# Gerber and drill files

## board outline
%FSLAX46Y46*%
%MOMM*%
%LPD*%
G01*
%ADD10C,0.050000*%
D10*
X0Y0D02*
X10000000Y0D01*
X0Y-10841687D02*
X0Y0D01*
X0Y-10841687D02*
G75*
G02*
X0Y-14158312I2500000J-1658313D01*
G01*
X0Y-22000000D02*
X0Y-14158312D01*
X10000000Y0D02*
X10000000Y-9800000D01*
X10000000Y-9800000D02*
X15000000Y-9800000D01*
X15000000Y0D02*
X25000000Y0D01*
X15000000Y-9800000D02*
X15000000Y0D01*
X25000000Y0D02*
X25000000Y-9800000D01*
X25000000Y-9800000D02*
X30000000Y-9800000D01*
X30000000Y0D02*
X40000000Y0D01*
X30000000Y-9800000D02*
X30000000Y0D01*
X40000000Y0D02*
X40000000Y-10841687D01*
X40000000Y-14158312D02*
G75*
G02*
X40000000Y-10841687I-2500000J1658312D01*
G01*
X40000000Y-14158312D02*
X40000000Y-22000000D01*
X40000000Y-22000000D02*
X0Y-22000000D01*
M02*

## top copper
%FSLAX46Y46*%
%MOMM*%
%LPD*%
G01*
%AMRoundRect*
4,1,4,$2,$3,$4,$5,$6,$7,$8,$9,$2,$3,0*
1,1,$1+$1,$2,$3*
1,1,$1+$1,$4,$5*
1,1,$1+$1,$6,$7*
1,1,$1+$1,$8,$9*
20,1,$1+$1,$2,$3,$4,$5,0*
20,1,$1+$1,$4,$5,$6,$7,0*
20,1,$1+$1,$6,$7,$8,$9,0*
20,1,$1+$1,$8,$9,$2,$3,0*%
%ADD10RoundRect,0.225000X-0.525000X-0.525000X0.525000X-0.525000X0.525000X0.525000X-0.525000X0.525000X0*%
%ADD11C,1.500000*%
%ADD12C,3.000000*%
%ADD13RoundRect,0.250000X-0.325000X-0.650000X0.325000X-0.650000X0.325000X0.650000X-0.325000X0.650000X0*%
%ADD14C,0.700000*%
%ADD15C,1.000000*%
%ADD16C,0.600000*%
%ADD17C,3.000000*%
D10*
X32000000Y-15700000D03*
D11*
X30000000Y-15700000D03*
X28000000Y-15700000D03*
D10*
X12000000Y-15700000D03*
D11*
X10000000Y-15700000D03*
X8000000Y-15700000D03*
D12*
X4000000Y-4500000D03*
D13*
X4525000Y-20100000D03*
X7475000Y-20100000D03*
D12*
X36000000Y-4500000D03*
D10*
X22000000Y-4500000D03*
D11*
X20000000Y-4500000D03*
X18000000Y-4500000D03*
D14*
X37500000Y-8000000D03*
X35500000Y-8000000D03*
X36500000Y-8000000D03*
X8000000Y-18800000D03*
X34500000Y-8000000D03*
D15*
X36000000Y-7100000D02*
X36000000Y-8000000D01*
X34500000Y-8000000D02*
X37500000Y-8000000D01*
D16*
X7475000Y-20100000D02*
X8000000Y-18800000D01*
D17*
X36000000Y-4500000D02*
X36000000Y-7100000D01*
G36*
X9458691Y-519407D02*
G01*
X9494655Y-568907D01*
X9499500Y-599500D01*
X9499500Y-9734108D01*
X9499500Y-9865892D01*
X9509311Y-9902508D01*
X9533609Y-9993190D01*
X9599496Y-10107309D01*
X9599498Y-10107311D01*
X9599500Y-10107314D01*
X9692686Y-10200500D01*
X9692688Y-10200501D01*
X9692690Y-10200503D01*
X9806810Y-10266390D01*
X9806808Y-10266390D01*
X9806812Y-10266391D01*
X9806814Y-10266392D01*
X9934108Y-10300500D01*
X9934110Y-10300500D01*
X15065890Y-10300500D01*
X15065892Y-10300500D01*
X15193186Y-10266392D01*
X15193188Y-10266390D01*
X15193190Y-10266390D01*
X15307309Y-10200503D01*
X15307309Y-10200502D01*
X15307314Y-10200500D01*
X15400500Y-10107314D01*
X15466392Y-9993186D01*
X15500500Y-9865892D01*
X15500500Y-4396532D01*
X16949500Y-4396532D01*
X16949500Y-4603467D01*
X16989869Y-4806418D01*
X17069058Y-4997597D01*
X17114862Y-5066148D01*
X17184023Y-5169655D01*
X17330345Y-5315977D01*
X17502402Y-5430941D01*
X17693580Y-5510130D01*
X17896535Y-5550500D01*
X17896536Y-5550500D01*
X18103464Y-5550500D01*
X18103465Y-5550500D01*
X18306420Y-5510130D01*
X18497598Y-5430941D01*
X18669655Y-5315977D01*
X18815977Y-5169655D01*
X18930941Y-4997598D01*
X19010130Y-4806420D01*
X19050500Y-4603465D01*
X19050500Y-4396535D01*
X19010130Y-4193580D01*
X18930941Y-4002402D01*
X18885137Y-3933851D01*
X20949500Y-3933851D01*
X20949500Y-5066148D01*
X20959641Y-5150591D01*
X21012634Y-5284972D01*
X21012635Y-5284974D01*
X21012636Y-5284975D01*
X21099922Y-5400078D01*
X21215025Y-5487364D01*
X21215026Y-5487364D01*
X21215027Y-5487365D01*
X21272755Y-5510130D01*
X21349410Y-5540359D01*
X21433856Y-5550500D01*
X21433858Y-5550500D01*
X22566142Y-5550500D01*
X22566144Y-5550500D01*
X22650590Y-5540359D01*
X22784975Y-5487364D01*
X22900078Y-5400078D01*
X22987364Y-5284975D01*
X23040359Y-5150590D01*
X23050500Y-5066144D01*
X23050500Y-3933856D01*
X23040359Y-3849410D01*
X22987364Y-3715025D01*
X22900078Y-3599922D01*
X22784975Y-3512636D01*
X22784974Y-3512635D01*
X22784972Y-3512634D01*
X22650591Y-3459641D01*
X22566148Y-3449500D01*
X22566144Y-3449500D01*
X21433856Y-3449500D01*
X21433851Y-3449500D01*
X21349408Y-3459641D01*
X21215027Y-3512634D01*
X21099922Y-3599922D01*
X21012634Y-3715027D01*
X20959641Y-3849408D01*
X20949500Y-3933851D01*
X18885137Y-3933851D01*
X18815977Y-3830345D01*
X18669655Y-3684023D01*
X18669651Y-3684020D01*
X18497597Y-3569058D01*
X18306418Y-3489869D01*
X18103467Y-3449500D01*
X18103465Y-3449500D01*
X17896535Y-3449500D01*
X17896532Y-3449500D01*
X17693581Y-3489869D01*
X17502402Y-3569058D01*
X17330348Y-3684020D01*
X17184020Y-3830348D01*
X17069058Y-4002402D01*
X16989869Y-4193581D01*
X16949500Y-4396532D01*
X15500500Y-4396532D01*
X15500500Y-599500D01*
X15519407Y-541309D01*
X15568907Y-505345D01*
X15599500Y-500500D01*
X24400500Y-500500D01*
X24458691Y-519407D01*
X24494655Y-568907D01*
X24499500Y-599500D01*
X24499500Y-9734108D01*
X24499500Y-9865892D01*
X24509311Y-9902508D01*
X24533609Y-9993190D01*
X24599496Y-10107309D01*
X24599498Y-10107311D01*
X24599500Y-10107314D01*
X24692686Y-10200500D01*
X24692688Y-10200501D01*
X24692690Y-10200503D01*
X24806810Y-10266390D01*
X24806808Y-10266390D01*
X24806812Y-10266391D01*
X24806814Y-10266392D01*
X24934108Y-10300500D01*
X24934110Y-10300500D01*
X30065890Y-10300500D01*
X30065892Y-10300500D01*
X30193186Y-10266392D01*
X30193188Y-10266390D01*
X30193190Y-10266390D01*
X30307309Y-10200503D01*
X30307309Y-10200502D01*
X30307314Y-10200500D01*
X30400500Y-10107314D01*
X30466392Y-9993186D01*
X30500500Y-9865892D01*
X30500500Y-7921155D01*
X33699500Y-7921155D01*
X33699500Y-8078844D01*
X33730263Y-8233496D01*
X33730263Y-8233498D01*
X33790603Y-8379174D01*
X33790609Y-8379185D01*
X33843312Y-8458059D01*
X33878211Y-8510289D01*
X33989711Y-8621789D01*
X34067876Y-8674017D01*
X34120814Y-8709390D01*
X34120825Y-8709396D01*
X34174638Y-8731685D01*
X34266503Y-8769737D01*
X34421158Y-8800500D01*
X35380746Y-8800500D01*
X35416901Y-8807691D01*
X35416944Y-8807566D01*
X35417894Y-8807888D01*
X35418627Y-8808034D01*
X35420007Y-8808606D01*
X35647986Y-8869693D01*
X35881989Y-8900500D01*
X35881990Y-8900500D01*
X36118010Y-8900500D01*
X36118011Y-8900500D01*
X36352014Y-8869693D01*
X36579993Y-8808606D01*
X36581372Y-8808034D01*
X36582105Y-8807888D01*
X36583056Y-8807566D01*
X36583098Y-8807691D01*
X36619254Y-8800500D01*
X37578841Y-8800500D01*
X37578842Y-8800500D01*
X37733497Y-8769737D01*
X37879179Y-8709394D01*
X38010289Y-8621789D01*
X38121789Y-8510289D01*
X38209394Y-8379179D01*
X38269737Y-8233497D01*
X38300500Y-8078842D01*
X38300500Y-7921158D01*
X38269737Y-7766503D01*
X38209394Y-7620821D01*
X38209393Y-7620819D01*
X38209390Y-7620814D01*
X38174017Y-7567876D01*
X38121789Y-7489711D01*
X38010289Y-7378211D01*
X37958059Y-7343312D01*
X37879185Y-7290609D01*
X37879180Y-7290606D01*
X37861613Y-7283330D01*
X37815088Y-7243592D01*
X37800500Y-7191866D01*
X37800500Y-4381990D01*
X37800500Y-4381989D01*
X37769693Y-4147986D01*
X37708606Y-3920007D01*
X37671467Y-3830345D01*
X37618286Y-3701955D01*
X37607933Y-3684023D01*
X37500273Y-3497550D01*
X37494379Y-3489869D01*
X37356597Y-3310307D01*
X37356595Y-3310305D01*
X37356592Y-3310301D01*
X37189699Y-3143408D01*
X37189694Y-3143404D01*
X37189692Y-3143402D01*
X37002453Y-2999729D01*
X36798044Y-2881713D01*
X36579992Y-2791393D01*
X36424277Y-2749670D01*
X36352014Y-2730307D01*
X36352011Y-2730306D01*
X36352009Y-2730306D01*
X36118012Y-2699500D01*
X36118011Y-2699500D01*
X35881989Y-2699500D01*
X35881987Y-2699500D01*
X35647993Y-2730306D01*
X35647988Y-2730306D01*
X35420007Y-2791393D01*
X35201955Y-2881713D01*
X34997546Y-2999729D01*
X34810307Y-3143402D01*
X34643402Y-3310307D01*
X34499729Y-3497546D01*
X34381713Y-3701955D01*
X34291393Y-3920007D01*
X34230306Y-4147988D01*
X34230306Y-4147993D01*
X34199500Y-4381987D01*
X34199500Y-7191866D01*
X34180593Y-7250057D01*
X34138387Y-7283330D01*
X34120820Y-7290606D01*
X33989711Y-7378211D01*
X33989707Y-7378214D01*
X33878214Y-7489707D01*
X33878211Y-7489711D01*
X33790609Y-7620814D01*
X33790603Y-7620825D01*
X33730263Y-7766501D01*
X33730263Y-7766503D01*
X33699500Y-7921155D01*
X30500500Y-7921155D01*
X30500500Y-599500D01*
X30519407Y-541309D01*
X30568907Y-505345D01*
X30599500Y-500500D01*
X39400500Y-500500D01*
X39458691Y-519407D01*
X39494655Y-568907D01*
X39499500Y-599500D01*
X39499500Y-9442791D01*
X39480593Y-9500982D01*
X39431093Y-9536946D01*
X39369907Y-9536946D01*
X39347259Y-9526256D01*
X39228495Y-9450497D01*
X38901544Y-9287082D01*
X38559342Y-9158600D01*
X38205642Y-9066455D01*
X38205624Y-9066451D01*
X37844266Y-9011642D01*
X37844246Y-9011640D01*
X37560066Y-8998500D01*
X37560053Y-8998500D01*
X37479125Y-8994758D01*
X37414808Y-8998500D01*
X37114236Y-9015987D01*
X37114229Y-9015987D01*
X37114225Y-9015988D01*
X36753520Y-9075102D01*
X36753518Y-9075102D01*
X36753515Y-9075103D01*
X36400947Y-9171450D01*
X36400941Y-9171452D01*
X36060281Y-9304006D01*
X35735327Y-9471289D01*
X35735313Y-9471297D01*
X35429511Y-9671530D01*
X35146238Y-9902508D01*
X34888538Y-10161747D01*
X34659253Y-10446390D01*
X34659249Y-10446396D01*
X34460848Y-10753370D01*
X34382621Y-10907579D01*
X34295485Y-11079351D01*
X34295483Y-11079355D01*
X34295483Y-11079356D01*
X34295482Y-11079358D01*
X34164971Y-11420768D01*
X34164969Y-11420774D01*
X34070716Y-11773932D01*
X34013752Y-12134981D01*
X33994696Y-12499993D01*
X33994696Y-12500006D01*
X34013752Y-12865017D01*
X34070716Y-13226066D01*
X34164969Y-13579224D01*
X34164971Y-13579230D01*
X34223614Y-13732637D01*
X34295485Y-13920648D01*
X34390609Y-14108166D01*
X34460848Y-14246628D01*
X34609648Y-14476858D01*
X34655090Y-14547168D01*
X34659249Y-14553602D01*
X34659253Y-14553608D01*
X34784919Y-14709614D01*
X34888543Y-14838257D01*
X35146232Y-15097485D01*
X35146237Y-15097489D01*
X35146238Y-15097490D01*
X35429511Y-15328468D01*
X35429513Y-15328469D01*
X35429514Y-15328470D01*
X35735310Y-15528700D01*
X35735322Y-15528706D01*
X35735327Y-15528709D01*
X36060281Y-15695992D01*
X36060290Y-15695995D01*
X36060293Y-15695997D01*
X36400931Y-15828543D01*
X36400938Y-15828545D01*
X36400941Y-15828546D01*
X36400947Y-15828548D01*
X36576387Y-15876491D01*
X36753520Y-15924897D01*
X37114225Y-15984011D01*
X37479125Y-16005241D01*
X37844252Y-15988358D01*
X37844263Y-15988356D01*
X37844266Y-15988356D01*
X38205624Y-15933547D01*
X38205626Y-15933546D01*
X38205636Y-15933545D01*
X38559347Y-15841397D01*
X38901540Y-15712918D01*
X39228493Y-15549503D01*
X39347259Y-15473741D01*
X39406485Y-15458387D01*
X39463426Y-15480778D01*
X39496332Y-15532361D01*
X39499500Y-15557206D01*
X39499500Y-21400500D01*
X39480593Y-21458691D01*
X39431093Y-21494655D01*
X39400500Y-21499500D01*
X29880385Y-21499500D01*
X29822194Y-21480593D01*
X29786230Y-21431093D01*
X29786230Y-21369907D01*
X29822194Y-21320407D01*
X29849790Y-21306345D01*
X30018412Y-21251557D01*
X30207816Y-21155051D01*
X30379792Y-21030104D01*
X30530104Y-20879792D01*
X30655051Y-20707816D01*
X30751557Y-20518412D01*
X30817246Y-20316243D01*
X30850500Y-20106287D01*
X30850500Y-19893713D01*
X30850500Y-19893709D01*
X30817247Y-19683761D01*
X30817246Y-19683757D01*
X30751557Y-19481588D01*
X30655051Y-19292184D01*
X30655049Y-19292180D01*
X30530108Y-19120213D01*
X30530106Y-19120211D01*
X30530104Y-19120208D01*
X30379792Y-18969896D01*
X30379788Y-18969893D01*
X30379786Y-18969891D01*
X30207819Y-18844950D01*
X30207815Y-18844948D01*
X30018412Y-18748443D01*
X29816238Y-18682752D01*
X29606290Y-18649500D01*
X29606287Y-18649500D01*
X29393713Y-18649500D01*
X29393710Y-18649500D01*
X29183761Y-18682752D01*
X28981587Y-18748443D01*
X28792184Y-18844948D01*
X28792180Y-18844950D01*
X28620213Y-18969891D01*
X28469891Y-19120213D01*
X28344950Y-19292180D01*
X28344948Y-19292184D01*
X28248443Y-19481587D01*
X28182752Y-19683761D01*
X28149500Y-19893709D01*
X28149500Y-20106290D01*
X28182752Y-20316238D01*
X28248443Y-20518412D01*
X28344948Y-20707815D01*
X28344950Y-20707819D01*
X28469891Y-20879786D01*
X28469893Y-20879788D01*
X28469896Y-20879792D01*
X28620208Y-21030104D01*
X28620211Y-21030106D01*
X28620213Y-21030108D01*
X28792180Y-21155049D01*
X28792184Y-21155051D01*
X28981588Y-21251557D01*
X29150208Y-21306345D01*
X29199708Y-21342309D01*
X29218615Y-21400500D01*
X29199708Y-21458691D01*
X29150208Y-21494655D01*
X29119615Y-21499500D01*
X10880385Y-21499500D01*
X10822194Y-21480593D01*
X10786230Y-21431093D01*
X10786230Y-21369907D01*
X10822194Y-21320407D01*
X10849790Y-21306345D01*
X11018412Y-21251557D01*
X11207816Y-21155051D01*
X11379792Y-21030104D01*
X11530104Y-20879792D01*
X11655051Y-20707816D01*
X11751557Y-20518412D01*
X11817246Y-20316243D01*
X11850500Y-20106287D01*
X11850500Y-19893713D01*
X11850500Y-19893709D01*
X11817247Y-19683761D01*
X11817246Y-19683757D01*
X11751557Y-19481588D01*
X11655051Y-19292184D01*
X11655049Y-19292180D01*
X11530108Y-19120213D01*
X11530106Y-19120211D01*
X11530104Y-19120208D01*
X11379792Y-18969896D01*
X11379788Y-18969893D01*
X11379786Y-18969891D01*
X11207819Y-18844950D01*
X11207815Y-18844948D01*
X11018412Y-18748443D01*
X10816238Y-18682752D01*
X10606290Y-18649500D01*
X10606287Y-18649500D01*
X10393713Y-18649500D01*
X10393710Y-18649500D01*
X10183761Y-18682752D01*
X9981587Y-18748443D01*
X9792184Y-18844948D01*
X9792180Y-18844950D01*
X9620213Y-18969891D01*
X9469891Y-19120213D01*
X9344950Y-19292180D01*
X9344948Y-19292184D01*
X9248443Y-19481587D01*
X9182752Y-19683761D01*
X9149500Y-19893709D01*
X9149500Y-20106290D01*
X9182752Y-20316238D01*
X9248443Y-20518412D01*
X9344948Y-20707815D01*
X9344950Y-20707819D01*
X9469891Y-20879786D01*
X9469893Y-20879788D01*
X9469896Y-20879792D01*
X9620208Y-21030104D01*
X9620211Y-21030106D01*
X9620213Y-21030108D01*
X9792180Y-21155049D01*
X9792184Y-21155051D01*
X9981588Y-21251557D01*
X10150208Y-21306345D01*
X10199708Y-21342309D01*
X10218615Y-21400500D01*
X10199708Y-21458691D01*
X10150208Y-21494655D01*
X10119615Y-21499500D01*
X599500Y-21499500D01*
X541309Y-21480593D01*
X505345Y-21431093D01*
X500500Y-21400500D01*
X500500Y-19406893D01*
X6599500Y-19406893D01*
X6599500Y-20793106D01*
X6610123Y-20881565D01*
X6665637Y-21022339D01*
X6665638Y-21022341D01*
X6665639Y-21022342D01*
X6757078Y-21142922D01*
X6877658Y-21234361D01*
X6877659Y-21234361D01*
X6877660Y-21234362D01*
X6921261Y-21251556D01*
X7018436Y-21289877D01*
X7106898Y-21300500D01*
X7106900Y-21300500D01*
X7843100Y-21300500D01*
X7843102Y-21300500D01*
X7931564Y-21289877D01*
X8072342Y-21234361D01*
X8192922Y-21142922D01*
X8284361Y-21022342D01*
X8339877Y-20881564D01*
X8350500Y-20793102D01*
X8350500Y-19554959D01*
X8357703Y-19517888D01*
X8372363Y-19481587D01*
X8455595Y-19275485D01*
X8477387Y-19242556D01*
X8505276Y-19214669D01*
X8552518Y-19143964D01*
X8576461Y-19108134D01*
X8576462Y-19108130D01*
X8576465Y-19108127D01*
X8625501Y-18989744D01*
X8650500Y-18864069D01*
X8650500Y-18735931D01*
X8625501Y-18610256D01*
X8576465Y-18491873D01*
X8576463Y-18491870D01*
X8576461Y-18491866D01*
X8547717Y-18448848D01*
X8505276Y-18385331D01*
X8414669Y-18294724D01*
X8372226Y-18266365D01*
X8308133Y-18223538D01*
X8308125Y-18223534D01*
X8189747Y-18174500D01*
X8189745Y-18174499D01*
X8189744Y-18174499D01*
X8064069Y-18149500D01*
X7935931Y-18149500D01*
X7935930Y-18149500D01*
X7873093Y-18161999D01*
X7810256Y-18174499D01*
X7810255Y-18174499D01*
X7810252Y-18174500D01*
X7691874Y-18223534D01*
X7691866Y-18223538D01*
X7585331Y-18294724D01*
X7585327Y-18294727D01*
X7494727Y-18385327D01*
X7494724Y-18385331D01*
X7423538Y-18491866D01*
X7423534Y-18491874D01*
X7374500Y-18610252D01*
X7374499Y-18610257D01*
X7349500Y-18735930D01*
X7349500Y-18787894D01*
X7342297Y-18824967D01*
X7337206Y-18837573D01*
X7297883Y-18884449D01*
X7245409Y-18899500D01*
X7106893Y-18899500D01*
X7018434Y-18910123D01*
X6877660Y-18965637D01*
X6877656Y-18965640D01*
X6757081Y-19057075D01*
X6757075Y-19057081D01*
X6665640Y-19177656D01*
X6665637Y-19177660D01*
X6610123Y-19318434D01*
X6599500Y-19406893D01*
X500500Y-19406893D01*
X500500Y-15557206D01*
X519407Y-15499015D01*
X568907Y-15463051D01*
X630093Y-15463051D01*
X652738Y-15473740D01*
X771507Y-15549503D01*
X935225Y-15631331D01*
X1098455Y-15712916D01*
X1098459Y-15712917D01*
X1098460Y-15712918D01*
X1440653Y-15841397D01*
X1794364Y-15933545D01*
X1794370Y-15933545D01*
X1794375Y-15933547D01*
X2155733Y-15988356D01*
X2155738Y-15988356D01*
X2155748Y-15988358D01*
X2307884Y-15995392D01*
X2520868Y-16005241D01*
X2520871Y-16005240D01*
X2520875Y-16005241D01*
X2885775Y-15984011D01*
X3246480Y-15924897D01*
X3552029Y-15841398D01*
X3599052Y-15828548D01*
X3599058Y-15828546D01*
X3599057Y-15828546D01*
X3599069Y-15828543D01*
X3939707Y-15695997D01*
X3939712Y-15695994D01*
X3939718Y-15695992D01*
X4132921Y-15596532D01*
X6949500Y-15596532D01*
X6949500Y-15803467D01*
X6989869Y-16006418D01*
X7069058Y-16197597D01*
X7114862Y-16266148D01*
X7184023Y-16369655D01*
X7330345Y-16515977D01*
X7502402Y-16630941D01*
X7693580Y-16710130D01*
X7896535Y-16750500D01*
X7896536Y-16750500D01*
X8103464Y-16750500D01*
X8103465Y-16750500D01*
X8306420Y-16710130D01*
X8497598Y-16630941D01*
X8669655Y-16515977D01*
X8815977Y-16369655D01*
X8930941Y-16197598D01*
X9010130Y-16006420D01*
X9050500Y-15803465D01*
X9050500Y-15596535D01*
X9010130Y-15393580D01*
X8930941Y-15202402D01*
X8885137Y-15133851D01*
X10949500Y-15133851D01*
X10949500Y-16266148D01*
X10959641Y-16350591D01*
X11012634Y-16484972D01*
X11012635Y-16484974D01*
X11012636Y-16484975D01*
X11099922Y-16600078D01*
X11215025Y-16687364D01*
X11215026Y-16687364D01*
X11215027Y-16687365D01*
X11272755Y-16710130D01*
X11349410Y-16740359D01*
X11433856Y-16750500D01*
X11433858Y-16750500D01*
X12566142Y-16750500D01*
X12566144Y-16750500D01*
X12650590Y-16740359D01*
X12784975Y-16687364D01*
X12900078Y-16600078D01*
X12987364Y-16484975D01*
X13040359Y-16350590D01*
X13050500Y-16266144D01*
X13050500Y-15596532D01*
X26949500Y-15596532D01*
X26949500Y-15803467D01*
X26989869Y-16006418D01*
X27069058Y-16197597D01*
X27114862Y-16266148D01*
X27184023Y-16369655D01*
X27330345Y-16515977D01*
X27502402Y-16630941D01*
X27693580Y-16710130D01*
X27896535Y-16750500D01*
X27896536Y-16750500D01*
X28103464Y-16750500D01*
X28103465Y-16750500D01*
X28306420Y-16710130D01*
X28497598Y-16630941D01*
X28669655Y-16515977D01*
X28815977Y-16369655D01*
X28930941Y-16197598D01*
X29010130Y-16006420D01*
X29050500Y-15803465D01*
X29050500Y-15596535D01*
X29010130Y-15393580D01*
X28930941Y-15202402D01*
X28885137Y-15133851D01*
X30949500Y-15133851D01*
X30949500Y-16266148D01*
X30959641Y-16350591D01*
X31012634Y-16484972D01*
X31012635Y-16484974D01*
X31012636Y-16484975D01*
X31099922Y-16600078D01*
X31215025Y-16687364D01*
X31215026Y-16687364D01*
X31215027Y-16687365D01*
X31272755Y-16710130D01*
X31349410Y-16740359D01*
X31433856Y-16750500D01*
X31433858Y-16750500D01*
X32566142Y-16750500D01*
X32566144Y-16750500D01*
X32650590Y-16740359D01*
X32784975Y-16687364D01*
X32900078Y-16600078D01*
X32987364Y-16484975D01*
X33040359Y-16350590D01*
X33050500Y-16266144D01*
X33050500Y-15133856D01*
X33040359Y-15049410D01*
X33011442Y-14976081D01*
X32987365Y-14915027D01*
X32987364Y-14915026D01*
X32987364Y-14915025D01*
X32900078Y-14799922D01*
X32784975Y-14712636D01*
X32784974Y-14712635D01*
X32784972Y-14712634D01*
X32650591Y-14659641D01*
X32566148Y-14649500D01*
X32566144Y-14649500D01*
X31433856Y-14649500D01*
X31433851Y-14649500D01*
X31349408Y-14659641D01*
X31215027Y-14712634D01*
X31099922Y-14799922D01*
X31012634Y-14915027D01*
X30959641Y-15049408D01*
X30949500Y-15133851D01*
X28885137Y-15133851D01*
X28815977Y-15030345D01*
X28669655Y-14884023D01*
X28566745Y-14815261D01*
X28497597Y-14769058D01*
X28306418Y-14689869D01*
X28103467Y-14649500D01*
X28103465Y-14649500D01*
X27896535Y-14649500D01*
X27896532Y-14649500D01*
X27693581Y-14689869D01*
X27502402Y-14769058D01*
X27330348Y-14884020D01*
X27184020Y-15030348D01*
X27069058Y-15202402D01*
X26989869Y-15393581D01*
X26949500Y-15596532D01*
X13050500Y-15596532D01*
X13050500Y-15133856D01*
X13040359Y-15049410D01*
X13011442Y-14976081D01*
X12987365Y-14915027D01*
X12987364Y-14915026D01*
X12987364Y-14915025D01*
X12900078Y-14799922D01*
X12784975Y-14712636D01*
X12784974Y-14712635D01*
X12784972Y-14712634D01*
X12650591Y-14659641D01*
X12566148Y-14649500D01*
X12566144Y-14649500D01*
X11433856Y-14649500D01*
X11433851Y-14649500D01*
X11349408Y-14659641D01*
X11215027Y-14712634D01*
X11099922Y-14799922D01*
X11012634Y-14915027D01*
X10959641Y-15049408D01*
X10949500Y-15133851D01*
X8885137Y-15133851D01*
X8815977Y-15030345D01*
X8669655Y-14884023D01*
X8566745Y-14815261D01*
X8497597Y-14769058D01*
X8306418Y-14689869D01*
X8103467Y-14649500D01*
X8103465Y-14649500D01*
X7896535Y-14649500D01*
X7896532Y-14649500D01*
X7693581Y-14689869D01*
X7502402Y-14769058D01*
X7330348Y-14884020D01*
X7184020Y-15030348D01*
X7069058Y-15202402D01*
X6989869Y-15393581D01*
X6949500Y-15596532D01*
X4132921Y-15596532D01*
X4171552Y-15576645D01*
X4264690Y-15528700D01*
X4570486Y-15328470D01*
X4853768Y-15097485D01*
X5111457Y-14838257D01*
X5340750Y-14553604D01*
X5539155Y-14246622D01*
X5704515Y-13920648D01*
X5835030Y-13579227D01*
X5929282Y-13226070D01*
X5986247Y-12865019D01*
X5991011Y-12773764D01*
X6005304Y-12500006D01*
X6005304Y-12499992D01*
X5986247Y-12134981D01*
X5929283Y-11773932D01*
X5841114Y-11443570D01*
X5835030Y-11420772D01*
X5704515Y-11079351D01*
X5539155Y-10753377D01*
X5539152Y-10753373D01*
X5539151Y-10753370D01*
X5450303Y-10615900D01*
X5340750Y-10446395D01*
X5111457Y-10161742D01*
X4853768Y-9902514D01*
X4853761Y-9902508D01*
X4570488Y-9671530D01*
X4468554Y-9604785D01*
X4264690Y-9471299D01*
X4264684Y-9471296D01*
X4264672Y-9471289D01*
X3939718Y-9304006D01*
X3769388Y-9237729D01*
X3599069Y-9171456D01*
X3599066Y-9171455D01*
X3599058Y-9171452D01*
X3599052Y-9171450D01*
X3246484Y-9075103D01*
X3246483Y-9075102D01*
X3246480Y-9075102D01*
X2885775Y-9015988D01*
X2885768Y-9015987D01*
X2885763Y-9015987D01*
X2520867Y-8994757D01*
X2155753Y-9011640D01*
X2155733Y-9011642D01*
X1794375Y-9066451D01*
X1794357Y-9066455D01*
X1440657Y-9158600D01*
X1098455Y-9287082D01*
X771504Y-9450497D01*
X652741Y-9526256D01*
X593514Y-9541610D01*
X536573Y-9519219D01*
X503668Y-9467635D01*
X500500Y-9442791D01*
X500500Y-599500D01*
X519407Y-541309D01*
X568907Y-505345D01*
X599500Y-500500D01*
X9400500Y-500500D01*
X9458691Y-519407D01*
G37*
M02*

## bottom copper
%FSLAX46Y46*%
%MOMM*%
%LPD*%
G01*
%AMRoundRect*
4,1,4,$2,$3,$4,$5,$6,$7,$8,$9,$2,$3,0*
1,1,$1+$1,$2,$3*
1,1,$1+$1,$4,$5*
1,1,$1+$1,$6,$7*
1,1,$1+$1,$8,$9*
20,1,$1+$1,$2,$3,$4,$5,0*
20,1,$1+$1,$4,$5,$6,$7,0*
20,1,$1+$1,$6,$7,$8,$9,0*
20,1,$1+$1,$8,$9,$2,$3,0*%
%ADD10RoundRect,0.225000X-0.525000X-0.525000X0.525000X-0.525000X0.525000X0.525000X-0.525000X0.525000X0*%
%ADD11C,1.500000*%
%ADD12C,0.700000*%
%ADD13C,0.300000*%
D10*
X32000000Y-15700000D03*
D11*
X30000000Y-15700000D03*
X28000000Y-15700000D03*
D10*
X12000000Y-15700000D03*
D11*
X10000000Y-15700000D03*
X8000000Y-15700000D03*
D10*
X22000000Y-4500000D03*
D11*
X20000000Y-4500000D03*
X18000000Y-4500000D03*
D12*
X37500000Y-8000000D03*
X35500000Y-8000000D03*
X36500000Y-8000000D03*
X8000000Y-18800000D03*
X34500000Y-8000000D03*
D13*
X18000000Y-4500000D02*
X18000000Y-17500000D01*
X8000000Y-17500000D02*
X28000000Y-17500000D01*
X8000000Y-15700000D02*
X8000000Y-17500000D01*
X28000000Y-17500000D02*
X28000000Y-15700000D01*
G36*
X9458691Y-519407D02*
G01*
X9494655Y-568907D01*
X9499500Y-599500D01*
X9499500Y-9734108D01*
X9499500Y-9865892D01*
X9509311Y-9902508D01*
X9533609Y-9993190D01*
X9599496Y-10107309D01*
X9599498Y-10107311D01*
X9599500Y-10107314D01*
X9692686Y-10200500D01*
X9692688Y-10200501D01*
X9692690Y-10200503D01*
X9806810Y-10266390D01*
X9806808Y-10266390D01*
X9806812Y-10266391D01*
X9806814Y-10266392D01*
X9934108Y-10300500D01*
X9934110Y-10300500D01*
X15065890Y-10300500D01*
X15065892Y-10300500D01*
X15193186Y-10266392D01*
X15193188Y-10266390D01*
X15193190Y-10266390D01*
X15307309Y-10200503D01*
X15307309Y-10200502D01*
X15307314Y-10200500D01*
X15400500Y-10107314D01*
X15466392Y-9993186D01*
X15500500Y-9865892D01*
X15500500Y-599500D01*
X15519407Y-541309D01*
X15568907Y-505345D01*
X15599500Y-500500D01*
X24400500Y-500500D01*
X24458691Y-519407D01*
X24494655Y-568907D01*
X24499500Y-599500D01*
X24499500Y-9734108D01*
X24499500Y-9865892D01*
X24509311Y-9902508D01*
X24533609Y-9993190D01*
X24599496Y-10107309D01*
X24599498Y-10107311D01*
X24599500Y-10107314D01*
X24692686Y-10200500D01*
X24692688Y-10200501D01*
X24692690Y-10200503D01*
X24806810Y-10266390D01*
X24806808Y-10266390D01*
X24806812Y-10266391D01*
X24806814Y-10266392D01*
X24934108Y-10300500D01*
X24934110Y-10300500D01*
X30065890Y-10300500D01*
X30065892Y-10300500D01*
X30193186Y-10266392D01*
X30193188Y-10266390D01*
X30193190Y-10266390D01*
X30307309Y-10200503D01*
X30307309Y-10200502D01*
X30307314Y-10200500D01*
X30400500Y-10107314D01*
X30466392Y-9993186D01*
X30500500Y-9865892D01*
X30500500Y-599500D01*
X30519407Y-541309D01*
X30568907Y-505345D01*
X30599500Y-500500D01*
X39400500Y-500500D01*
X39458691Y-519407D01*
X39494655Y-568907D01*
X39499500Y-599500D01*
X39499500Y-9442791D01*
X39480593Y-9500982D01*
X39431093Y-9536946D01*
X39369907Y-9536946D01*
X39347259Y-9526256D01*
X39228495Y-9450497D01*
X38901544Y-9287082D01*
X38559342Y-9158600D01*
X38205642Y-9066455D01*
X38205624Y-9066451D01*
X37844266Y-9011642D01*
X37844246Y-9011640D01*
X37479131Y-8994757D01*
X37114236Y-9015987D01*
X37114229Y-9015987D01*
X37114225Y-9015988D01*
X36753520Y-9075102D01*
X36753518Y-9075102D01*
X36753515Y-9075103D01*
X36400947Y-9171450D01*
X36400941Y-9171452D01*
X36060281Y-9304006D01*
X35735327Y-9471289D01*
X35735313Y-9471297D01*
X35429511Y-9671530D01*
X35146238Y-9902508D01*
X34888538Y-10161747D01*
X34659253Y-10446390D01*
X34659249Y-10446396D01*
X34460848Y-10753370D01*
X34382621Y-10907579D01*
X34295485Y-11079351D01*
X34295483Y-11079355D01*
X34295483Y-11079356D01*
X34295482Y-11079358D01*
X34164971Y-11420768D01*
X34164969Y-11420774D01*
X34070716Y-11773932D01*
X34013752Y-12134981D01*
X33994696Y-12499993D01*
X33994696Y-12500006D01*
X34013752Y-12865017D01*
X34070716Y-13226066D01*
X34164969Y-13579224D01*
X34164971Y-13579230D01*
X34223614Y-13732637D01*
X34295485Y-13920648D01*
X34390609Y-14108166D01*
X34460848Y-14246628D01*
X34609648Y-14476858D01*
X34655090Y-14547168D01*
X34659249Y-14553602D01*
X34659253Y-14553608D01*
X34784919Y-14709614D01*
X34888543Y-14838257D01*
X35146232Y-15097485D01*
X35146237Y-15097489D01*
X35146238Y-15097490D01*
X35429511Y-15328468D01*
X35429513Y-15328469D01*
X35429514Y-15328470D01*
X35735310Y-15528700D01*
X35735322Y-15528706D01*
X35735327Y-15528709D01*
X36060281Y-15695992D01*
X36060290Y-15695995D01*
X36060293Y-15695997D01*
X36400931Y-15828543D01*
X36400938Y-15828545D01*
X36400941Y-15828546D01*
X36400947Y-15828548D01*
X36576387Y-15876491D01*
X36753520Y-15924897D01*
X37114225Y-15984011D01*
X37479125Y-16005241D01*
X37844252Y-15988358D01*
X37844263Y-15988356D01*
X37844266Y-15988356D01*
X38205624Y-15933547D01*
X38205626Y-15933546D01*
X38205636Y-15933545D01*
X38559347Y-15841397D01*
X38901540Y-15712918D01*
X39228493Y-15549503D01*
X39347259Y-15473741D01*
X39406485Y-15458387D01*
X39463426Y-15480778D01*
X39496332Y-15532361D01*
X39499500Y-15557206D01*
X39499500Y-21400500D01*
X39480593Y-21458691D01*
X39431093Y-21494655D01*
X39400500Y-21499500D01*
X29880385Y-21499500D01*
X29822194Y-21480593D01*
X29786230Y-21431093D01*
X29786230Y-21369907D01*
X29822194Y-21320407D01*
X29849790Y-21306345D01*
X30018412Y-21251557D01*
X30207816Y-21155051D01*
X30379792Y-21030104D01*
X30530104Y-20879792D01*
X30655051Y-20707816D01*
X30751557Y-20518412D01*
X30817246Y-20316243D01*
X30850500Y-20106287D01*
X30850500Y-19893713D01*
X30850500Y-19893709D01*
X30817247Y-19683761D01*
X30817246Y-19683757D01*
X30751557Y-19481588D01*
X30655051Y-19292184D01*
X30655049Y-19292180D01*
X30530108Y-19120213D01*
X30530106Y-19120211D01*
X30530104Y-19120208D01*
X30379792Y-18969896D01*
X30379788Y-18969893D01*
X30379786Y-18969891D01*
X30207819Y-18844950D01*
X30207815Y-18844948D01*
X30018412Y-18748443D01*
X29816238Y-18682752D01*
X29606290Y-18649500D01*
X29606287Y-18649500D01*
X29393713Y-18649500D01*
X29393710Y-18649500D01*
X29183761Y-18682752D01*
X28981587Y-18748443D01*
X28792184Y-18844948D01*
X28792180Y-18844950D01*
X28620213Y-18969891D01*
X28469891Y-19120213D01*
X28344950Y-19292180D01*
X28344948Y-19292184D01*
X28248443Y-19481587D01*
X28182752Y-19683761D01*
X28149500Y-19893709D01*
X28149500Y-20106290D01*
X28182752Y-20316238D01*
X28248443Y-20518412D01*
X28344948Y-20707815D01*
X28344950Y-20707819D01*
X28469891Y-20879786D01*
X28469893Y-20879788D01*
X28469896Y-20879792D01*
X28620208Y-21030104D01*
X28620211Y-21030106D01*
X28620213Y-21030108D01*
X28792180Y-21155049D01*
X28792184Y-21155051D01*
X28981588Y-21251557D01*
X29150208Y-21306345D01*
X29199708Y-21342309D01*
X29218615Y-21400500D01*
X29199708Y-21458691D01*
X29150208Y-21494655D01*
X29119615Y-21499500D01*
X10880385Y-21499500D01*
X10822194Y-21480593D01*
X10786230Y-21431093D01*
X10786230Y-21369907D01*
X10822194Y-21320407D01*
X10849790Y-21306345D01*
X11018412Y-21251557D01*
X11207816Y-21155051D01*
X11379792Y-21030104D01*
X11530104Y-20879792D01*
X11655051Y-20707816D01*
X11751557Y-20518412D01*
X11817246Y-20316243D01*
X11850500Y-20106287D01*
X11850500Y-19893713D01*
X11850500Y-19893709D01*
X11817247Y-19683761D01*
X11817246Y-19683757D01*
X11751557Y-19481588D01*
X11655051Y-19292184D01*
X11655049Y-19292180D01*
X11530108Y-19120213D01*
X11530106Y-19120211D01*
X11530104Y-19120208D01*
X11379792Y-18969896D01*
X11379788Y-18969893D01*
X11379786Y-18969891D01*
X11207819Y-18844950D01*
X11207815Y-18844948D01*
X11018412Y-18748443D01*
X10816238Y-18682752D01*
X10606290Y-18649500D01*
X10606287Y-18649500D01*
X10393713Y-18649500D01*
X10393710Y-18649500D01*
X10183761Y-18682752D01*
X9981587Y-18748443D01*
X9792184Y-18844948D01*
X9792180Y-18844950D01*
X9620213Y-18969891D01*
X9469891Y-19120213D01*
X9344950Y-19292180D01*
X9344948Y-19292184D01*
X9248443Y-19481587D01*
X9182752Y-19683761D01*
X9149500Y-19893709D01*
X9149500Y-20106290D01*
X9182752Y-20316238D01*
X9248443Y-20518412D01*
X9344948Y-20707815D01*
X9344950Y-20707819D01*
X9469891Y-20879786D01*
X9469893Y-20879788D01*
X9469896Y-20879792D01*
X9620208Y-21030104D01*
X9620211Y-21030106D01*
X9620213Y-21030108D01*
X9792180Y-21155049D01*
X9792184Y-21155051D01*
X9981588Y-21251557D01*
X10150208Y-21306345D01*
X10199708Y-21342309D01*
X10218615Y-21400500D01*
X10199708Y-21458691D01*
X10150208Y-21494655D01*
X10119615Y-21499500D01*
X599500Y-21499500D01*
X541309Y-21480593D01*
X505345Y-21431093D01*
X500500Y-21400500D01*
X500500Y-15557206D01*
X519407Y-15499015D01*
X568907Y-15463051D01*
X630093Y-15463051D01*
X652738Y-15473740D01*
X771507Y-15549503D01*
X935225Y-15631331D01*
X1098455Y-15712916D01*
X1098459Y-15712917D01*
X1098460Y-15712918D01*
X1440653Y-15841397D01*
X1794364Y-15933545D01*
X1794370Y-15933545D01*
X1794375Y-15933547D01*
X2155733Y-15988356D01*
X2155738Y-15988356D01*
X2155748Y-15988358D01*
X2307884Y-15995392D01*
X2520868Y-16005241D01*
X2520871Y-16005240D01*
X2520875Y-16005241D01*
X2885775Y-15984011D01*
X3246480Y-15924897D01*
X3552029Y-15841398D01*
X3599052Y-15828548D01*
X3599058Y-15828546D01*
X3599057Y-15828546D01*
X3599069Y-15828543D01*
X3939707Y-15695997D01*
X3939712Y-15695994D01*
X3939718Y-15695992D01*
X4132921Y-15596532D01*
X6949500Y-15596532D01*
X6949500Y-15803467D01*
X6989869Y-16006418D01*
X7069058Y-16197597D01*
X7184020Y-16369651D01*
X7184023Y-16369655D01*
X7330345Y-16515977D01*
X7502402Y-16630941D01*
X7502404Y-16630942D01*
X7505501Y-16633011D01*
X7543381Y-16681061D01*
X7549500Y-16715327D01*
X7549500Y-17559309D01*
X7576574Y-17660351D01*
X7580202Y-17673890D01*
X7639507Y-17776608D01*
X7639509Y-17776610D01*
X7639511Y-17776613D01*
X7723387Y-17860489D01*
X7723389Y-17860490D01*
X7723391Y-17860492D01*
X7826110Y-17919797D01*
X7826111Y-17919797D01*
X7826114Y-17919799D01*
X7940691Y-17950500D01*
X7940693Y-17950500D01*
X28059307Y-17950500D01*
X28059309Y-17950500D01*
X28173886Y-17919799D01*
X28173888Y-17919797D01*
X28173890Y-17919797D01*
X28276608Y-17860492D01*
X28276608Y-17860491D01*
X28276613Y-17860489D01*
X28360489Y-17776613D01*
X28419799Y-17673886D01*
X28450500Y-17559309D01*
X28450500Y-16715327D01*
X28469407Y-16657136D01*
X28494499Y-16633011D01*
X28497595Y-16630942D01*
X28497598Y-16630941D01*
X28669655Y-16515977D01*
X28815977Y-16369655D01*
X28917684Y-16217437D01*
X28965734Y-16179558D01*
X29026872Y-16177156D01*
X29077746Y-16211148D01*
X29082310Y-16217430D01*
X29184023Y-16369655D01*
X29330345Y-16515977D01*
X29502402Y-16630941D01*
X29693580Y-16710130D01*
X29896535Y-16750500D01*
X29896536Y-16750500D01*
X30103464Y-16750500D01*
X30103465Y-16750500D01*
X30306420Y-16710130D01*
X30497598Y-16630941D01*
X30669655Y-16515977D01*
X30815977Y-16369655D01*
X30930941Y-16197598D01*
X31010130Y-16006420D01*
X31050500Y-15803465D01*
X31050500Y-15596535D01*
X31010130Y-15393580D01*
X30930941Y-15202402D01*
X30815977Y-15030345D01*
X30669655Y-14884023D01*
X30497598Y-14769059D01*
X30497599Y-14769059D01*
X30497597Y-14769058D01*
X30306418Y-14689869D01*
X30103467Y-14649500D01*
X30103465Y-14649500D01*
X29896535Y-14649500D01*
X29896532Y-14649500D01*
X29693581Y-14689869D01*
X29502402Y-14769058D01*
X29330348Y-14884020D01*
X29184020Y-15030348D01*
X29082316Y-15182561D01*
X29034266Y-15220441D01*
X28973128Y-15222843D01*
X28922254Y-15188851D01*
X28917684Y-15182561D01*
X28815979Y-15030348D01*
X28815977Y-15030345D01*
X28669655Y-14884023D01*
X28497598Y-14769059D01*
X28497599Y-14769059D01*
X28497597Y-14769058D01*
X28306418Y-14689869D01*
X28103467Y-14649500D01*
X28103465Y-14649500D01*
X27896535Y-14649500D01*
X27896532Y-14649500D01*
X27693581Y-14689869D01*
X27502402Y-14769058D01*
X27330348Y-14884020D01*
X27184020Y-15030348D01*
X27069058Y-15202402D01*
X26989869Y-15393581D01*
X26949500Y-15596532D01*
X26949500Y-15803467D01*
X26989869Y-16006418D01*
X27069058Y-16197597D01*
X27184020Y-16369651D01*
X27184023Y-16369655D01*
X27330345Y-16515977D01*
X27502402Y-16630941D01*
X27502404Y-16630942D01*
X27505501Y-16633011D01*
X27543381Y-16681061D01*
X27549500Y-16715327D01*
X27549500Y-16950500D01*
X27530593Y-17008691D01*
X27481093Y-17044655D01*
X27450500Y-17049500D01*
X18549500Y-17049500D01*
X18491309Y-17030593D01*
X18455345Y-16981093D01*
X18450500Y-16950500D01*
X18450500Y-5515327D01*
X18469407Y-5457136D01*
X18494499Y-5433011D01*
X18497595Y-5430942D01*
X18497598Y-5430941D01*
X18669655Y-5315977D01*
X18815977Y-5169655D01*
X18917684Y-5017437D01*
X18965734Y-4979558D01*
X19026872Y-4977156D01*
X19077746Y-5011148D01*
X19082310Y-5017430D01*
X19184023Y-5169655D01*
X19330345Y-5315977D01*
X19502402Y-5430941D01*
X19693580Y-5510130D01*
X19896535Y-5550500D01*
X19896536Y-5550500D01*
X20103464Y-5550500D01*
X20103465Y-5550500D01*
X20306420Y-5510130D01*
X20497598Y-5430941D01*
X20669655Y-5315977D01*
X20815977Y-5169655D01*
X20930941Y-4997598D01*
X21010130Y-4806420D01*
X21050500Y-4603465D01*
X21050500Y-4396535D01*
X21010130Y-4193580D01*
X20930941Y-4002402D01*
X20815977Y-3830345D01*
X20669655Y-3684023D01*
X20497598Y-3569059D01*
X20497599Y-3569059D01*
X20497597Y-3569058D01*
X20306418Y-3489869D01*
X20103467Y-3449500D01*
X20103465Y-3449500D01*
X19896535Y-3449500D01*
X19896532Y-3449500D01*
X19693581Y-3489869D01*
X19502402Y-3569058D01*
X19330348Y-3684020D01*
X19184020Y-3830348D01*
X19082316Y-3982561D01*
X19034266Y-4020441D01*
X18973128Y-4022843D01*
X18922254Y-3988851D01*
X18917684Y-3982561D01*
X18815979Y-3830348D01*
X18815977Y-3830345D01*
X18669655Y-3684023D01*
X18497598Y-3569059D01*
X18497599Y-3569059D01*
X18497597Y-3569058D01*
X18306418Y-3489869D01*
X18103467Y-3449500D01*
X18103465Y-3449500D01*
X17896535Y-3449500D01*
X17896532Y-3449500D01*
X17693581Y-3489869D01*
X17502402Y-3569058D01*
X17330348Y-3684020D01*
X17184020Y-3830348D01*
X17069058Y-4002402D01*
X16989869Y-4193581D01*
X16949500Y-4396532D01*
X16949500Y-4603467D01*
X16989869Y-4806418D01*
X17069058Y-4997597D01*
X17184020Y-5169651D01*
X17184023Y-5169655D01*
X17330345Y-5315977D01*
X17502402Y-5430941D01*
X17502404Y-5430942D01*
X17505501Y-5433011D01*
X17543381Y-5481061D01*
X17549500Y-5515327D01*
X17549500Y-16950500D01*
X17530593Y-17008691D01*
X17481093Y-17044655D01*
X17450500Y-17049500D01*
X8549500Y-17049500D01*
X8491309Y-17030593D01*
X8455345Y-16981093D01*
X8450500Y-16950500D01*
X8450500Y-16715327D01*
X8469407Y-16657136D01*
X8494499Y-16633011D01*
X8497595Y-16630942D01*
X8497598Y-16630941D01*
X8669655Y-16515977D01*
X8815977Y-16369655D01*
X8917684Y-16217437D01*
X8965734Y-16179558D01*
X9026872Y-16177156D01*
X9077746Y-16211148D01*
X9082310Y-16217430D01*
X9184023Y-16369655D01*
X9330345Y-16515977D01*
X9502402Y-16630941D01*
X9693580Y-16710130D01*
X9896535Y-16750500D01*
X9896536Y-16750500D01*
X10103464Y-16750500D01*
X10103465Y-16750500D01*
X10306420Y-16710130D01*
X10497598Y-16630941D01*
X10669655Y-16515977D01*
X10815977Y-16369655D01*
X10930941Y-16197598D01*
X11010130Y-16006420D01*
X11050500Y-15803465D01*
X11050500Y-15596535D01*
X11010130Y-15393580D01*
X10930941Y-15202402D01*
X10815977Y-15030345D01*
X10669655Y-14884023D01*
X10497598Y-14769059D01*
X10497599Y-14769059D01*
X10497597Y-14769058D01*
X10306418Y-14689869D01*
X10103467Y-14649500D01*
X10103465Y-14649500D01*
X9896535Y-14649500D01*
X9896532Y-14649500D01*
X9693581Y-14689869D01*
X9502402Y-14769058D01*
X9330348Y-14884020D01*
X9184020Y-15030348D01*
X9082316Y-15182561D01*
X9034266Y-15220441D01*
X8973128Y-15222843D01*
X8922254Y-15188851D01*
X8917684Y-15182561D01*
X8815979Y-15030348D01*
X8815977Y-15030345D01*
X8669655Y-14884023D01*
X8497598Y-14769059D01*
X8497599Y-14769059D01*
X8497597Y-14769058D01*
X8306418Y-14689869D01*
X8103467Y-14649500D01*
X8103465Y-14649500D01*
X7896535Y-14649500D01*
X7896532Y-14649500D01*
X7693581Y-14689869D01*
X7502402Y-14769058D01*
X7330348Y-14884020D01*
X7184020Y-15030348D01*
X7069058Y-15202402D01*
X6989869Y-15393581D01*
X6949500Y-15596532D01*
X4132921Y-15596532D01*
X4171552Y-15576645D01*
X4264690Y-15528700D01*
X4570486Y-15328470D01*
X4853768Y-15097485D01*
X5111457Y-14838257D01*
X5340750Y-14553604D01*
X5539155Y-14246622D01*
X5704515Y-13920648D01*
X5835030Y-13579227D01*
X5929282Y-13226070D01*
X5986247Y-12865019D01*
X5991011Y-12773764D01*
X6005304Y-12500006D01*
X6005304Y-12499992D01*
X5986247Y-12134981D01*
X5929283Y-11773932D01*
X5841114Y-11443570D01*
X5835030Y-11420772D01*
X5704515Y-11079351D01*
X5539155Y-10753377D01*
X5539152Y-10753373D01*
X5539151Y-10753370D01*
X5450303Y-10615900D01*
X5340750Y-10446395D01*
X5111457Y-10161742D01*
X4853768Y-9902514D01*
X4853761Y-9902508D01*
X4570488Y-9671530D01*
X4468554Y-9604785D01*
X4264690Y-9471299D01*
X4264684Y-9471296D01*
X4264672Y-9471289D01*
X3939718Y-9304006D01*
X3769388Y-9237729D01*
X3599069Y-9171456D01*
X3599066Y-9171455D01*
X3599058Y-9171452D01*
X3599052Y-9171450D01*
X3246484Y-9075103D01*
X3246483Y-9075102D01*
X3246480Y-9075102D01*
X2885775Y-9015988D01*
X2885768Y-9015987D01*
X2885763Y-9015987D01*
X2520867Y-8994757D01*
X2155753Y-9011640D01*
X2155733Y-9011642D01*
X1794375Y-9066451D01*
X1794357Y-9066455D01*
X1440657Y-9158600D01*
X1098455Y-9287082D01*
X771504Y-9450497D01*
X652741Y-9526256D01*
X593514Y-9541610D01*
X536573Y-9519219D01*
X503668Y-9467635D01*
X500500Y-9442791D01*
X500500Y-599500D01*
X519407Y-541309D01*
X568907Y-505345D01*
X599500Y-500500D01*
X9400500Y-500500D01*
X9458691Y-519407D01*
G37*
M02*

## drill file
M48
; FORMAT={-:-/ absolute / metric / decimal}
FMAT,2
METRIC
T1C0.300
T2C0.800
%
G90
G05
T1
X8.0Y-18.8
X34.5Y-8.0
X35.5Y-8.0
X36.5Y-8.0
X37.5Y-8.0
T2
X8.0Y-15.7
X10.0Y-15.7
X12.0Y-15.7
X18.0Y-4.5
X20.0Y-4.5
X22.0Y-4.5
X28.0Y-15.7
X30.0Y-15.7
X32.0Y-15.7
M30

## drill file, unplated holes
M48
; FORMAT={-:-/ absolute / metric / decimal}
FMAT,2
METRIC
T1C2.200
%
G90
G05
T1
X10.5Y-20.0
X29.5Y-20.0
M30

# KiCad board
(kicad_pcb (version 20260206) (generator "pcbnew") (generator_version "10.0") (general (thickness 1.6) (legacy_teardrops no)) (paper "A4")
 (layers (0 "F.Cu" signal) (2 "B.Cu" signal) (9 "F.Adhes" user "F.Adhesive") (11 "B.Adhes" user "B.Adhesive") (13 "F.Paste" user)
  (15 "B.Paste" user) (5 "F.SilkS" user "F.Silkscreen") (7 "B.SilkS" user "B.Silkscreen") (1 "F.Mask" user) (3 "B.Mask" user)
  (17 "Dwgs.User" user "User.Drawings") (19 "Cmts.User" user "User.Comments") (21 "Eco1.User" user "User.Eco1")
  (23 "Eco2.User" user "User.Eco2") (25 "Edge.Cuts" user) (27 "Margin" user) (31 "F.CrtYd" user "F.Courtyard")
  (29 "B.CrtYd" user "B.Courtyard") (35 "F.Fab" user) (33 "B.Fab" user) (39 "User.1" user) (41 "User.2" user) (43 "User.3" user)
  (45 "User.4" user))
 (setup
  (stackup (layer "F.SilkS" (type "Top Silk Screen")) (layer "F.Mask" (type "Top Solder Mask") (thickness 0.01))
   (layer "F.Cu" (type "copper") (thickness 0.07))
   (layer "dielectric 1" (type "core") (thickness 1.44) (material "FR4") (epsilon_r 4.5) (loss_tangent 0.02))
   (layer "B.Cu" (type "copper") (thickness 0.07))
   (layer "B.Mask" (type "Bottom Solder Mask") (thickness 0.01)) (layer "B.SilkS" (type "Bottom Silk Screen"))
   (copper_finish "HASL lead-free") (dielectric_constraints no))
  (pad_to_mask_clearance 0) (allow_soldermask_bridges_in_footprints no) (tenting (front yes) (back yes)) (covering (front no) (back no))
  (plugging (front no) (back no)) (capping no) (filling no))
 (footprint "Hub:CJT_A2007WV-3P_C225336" (layer "F.Cu") (at 28 15.7)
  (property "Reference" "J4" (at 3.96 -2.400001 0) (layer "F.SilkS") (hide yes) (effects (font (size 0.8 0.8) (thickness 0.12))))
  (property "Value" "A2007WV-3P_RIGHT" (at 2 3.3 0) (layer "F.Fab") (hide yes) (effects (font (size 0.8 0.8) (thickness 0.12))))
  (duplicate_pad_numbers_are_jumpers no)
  (pad "1" thru_hole roundrect (at 4 0) (size 1.5 1.5) (drill 0.8) (layers "*.Cu" "*.Mask") (remove_unused_layers no)
   (roundrect_rratio 0.15) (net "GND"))
  (pad "2" thru_hole circle (at 2 0) (size 1.5 1.5) (drill 0.8) (layers "*.Cu" "*.Mask") (remove_unused_layers no) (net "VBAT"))
  (pad "3" thru_hole circle (at 0 0) (size 1.5 1.5) (drill 0.8) (layers "*.Cu" "*.Mask") (remove_unused_layers no) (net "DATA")))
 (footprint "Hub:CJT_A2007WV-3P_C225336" (layer "F.Cu") (at 8 15.7)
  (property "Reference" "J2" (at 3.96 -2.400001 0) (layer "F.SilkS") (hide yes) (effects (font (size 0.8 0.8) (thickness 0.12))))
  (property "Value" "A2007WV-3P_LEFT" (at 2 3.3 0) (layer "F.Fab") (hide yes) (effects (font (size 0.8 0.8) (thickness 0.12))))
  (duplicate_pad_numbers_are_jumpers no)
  (pad "1" thru_hole roundrect (at 4 0) (size 1.5 1.5) (drill 0.8) (layers "*.Cu" "*.Mask") (remove_unused_layers no)
   (roundrect_rratio 0.15) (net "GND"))
  (pad "2" thru_hole circle (at 2 0) (size 1.5 1.5) (drill 0.8) (layers "*.Cu" "*.Mask") (remove_unused_layers no) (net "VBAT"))
  (pad "3" thru_hole circle (at 0 0) (size 1.5 1.5) (drill 0.8) (layers "*.Cu" "*.Mask") (remove_unused_layers no) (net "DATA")))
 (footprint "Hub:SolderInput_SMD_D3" (layer "F.Cu") (at 4 4.5)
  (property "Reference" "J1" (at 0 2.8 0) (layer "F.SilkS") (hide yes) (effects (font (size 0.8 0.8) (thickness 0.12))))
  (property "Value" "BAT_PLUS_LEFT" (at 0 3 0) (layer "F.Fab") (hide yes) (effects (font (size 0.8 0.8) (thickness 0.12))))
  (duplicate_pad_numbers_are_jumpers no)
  (pad "1" smd circle (at 0 0) (size 3 3) (layers "F.Cu" "F.Mask") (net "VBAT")))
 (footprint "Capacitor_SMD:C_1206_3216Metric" (layer "F.Cu") (at 6 20.1)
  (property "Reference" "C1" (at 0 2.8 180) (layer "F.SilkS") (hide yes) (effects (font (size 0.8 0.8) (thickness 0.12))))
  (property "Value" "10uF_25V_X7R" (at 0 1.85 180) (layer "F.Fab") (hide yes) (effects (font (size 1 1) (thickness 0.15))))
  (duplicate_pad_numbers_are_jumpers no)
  (pad "1" smd roundrect (at -1.475 0) (size 1.15 1.8) (layers "F.Cu" "F.Mask" "F.Paste") (roundrect_rratio 0.217391) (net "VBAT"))
  (pad "2" smd roundrect (at 1.475 0) (size 1.15 1.8) (layers "F.Cu" "F.Mask" "F.Paste") (roundrect_rratio 0.217391) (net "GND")))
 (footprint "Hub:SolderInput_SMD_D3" (layer "F.Cu") (at 36 4.5)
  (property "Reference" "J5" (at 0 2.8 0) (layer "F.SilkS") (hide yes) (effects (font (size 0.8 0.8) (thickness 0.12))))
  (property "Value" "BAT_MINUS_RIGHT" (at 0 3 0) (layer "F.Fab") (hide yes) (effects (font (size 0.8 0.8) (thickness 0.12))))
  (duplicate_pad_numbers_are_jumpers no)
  (pad "1" smd circle (at 0 0) (size 3 3) (layers "F.Cu" "F.Mask") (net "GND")))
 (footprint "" (layer "F.Cu") (at 10.5 20)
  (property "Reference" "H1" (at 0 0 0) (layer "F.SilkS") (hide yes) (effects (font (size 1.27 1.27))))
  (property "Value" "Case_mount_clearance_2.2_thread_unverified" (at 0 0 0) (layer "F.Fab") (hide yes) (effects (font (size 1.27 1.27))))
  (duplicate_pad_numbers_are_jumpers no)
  (pad "" np_thru_hole circle (at 0 0) (size 2.2 2.2) (drill 2.2) (layers "*.Cu")))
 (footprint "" (layer "F.Cu") (at 29.5 20)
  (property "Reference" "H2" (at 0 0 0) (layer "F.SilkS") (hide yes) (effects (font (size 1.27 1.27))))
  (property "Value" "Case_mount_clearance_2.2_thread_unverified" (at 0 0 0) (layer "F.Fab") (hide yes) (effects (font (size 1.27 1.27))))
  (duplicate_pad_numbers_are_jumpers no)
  (pad "" np_thru_hole circle (at 0 0) (size 2.2 2.2) (drill 2.2) (layers "*.Cu")))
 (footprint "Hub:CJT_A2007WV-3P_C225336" (layer "F.Cu") (at 18 4.5)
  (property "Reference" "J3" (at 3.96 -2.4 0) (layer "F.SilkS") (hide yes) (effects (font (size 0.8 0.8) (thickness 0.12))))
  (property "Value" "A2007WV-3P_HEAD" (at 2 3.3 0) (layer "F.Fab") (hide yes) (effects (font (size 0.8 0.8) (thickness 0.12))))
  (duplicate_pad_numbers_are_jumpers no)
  (pad "1" thru_hole roundrect (at 4 0) (size 1.5 1.5) (drill 0.8) (layers "*.Cu" "*.Mask") (remove_unused_layers no)
   (roundrect_rratio 0.15) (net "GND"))
  (pad "2" thru_hole circle (at 2 0) (size 1.5 1.5) (drill 0.8) (layers "*.Cu" "*.Mask") (remove_unused_layers no) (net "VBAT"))
  (pad "3" thru_hole circle (at 0 0) (size 1.5 1.5) (drill 0.8) (layers "*.Cu" "*.Mask") (remove_unused_layers no) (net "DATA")))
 (gr_line (start 0 0) (end 10 0) (stroke (width 0.05) (type default)) (layer "Edge.Cuts"))
 (gr_line (start 0 10.841687) (end 0 0) (stroke (width 0.05) (type default)) (layer "Edge.Cuts"))
 (gr_arc (start 0 10.841687) (mid 5.5 12.5) (end 0 14.158312) (stroke (width 0.05) (type default)) (layer "Edge.Cuts"))
 (gr_line (start 0 22) (end 0 14.158312) (stroke (width 0.05) (type default)) (layer "Edge.Cuts"))
 (gr_line (start 10 0) (end 10 9.8) (stroke (width 0.05) (type default)) (layer "Edge.Cuts"))
 (gr_line (start 10 9.8) (end 15 9.8) (stroke (width 0.05) (type default)) (layer "Edge.Cuts"))
 (gr_line (start 15 0) (end 25 0) (stroke (width 0.05) (type default)) (layer "Edge.Cuts"))
 (gr_line (start 15 9.8) (end 15 0) (stroke (width 0.05) (type default)) (layer "Edge.Cuts"))
 (gr_line (start 25 0) (end 25 9.8) (stroke (width 0.05) (type default)) (layer "Edge.Cuts"))
 (gr_line (start 25 9.8) (end 30 9.8) (stroke (width 0.05) (type default)) (layer "Edge.Cuts"))
 (gr_line (start 30 0) (end 40 0) (stroke (width 0.05) (type default)) (layer "Edge.Cuts"))
 (gr_line (start 30 9.8) (end 30 0) (stroke (width 0.05) (type default)) (layer "Edge.Cuts"))
 (gr_line (start 40 0) (end 40 10.841687) (stroke (width 0.05) (type default)) (layer "Edge.Cuts"))
 (gr_arc (start 40 14.158312) (mid 34.5 12.5) (end 40 10.841687) (stroke (width 0.05) (type default)) (layer "Edge.Cuts"))
 (gr_line (start 40 14.158312) (end 40 22) (stroke (width 0.05) (type default)) (layer "Edge.Cuts"))
 (gr_line (start 40 22) (end 0 22) (stroke (width 0.05) (type default)) (layer "Edge.Cuts"))
 (segment (start 36 7.1) (end 36 8) (width 1) (layer "F.Cu") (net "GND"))
 (segment (start 34.5 8) (end 37.5 8) (width 1) (layer "F.Cu") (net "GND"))
 (segment (start 7.475 20.1) (end 8 18.8) (width 0.6) (layer "F.Cu") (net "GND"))
 (segment (start 36 4.5) (end 36 7.1) (width 3) (layer "F.Cu") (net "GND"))
 (via (at 37.5 8) (size 0.7) (drill 0.3) (layers "F.Cu" "B.Cu") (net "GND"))
 (via (at 35.5 8) (size 0.7) (drill 0.3) (layers "F.Cu" "B.Cu") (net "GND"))
 (via (at 36.5 8) (size 0.7) (drill 0.3) (layers "F.Cu" "B.Cu") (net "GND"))
 (via (at 8 18.8) (size 0.7) (drill 0.3) (layers "F.Cu" "B.Cu") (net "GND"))
 (via (at 34.5 8) (size 0.7) (drill 0.3) (layers "F.Cu" "B.Cu") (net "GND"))
 (segment (start 18 4.5) (end 18 17.5) (width 0.3) (layer "B.Cu") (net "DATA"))
 (segment (start 8 17.5) (end 28 17.5) (width 0.3) (layer "B.Cu") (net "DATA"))
 (segment (start 8 15.7) (end 8 17.5) (width 0.3) (layer "B.Cu") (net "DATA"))
 (segment (start 28 17.5) (end 28 15.7) (width 0.3) (layer "B.Cu") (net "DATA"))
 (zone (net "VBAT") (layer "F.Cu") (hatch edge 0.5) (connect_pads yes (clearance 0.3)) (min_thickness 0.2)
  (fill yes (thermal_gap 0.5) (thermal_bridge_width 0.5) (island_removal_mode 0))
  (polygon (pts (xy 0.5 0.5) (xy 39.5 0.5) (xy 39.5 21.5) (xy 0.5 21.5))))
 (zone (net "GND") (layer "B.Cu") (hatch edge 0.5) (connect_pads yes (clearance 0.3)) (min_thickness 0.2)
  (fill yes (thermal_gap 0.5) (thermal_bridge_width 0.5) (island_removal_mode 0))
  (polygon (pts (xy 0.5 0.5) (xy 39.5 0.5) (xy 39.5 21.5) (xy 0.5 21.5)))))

